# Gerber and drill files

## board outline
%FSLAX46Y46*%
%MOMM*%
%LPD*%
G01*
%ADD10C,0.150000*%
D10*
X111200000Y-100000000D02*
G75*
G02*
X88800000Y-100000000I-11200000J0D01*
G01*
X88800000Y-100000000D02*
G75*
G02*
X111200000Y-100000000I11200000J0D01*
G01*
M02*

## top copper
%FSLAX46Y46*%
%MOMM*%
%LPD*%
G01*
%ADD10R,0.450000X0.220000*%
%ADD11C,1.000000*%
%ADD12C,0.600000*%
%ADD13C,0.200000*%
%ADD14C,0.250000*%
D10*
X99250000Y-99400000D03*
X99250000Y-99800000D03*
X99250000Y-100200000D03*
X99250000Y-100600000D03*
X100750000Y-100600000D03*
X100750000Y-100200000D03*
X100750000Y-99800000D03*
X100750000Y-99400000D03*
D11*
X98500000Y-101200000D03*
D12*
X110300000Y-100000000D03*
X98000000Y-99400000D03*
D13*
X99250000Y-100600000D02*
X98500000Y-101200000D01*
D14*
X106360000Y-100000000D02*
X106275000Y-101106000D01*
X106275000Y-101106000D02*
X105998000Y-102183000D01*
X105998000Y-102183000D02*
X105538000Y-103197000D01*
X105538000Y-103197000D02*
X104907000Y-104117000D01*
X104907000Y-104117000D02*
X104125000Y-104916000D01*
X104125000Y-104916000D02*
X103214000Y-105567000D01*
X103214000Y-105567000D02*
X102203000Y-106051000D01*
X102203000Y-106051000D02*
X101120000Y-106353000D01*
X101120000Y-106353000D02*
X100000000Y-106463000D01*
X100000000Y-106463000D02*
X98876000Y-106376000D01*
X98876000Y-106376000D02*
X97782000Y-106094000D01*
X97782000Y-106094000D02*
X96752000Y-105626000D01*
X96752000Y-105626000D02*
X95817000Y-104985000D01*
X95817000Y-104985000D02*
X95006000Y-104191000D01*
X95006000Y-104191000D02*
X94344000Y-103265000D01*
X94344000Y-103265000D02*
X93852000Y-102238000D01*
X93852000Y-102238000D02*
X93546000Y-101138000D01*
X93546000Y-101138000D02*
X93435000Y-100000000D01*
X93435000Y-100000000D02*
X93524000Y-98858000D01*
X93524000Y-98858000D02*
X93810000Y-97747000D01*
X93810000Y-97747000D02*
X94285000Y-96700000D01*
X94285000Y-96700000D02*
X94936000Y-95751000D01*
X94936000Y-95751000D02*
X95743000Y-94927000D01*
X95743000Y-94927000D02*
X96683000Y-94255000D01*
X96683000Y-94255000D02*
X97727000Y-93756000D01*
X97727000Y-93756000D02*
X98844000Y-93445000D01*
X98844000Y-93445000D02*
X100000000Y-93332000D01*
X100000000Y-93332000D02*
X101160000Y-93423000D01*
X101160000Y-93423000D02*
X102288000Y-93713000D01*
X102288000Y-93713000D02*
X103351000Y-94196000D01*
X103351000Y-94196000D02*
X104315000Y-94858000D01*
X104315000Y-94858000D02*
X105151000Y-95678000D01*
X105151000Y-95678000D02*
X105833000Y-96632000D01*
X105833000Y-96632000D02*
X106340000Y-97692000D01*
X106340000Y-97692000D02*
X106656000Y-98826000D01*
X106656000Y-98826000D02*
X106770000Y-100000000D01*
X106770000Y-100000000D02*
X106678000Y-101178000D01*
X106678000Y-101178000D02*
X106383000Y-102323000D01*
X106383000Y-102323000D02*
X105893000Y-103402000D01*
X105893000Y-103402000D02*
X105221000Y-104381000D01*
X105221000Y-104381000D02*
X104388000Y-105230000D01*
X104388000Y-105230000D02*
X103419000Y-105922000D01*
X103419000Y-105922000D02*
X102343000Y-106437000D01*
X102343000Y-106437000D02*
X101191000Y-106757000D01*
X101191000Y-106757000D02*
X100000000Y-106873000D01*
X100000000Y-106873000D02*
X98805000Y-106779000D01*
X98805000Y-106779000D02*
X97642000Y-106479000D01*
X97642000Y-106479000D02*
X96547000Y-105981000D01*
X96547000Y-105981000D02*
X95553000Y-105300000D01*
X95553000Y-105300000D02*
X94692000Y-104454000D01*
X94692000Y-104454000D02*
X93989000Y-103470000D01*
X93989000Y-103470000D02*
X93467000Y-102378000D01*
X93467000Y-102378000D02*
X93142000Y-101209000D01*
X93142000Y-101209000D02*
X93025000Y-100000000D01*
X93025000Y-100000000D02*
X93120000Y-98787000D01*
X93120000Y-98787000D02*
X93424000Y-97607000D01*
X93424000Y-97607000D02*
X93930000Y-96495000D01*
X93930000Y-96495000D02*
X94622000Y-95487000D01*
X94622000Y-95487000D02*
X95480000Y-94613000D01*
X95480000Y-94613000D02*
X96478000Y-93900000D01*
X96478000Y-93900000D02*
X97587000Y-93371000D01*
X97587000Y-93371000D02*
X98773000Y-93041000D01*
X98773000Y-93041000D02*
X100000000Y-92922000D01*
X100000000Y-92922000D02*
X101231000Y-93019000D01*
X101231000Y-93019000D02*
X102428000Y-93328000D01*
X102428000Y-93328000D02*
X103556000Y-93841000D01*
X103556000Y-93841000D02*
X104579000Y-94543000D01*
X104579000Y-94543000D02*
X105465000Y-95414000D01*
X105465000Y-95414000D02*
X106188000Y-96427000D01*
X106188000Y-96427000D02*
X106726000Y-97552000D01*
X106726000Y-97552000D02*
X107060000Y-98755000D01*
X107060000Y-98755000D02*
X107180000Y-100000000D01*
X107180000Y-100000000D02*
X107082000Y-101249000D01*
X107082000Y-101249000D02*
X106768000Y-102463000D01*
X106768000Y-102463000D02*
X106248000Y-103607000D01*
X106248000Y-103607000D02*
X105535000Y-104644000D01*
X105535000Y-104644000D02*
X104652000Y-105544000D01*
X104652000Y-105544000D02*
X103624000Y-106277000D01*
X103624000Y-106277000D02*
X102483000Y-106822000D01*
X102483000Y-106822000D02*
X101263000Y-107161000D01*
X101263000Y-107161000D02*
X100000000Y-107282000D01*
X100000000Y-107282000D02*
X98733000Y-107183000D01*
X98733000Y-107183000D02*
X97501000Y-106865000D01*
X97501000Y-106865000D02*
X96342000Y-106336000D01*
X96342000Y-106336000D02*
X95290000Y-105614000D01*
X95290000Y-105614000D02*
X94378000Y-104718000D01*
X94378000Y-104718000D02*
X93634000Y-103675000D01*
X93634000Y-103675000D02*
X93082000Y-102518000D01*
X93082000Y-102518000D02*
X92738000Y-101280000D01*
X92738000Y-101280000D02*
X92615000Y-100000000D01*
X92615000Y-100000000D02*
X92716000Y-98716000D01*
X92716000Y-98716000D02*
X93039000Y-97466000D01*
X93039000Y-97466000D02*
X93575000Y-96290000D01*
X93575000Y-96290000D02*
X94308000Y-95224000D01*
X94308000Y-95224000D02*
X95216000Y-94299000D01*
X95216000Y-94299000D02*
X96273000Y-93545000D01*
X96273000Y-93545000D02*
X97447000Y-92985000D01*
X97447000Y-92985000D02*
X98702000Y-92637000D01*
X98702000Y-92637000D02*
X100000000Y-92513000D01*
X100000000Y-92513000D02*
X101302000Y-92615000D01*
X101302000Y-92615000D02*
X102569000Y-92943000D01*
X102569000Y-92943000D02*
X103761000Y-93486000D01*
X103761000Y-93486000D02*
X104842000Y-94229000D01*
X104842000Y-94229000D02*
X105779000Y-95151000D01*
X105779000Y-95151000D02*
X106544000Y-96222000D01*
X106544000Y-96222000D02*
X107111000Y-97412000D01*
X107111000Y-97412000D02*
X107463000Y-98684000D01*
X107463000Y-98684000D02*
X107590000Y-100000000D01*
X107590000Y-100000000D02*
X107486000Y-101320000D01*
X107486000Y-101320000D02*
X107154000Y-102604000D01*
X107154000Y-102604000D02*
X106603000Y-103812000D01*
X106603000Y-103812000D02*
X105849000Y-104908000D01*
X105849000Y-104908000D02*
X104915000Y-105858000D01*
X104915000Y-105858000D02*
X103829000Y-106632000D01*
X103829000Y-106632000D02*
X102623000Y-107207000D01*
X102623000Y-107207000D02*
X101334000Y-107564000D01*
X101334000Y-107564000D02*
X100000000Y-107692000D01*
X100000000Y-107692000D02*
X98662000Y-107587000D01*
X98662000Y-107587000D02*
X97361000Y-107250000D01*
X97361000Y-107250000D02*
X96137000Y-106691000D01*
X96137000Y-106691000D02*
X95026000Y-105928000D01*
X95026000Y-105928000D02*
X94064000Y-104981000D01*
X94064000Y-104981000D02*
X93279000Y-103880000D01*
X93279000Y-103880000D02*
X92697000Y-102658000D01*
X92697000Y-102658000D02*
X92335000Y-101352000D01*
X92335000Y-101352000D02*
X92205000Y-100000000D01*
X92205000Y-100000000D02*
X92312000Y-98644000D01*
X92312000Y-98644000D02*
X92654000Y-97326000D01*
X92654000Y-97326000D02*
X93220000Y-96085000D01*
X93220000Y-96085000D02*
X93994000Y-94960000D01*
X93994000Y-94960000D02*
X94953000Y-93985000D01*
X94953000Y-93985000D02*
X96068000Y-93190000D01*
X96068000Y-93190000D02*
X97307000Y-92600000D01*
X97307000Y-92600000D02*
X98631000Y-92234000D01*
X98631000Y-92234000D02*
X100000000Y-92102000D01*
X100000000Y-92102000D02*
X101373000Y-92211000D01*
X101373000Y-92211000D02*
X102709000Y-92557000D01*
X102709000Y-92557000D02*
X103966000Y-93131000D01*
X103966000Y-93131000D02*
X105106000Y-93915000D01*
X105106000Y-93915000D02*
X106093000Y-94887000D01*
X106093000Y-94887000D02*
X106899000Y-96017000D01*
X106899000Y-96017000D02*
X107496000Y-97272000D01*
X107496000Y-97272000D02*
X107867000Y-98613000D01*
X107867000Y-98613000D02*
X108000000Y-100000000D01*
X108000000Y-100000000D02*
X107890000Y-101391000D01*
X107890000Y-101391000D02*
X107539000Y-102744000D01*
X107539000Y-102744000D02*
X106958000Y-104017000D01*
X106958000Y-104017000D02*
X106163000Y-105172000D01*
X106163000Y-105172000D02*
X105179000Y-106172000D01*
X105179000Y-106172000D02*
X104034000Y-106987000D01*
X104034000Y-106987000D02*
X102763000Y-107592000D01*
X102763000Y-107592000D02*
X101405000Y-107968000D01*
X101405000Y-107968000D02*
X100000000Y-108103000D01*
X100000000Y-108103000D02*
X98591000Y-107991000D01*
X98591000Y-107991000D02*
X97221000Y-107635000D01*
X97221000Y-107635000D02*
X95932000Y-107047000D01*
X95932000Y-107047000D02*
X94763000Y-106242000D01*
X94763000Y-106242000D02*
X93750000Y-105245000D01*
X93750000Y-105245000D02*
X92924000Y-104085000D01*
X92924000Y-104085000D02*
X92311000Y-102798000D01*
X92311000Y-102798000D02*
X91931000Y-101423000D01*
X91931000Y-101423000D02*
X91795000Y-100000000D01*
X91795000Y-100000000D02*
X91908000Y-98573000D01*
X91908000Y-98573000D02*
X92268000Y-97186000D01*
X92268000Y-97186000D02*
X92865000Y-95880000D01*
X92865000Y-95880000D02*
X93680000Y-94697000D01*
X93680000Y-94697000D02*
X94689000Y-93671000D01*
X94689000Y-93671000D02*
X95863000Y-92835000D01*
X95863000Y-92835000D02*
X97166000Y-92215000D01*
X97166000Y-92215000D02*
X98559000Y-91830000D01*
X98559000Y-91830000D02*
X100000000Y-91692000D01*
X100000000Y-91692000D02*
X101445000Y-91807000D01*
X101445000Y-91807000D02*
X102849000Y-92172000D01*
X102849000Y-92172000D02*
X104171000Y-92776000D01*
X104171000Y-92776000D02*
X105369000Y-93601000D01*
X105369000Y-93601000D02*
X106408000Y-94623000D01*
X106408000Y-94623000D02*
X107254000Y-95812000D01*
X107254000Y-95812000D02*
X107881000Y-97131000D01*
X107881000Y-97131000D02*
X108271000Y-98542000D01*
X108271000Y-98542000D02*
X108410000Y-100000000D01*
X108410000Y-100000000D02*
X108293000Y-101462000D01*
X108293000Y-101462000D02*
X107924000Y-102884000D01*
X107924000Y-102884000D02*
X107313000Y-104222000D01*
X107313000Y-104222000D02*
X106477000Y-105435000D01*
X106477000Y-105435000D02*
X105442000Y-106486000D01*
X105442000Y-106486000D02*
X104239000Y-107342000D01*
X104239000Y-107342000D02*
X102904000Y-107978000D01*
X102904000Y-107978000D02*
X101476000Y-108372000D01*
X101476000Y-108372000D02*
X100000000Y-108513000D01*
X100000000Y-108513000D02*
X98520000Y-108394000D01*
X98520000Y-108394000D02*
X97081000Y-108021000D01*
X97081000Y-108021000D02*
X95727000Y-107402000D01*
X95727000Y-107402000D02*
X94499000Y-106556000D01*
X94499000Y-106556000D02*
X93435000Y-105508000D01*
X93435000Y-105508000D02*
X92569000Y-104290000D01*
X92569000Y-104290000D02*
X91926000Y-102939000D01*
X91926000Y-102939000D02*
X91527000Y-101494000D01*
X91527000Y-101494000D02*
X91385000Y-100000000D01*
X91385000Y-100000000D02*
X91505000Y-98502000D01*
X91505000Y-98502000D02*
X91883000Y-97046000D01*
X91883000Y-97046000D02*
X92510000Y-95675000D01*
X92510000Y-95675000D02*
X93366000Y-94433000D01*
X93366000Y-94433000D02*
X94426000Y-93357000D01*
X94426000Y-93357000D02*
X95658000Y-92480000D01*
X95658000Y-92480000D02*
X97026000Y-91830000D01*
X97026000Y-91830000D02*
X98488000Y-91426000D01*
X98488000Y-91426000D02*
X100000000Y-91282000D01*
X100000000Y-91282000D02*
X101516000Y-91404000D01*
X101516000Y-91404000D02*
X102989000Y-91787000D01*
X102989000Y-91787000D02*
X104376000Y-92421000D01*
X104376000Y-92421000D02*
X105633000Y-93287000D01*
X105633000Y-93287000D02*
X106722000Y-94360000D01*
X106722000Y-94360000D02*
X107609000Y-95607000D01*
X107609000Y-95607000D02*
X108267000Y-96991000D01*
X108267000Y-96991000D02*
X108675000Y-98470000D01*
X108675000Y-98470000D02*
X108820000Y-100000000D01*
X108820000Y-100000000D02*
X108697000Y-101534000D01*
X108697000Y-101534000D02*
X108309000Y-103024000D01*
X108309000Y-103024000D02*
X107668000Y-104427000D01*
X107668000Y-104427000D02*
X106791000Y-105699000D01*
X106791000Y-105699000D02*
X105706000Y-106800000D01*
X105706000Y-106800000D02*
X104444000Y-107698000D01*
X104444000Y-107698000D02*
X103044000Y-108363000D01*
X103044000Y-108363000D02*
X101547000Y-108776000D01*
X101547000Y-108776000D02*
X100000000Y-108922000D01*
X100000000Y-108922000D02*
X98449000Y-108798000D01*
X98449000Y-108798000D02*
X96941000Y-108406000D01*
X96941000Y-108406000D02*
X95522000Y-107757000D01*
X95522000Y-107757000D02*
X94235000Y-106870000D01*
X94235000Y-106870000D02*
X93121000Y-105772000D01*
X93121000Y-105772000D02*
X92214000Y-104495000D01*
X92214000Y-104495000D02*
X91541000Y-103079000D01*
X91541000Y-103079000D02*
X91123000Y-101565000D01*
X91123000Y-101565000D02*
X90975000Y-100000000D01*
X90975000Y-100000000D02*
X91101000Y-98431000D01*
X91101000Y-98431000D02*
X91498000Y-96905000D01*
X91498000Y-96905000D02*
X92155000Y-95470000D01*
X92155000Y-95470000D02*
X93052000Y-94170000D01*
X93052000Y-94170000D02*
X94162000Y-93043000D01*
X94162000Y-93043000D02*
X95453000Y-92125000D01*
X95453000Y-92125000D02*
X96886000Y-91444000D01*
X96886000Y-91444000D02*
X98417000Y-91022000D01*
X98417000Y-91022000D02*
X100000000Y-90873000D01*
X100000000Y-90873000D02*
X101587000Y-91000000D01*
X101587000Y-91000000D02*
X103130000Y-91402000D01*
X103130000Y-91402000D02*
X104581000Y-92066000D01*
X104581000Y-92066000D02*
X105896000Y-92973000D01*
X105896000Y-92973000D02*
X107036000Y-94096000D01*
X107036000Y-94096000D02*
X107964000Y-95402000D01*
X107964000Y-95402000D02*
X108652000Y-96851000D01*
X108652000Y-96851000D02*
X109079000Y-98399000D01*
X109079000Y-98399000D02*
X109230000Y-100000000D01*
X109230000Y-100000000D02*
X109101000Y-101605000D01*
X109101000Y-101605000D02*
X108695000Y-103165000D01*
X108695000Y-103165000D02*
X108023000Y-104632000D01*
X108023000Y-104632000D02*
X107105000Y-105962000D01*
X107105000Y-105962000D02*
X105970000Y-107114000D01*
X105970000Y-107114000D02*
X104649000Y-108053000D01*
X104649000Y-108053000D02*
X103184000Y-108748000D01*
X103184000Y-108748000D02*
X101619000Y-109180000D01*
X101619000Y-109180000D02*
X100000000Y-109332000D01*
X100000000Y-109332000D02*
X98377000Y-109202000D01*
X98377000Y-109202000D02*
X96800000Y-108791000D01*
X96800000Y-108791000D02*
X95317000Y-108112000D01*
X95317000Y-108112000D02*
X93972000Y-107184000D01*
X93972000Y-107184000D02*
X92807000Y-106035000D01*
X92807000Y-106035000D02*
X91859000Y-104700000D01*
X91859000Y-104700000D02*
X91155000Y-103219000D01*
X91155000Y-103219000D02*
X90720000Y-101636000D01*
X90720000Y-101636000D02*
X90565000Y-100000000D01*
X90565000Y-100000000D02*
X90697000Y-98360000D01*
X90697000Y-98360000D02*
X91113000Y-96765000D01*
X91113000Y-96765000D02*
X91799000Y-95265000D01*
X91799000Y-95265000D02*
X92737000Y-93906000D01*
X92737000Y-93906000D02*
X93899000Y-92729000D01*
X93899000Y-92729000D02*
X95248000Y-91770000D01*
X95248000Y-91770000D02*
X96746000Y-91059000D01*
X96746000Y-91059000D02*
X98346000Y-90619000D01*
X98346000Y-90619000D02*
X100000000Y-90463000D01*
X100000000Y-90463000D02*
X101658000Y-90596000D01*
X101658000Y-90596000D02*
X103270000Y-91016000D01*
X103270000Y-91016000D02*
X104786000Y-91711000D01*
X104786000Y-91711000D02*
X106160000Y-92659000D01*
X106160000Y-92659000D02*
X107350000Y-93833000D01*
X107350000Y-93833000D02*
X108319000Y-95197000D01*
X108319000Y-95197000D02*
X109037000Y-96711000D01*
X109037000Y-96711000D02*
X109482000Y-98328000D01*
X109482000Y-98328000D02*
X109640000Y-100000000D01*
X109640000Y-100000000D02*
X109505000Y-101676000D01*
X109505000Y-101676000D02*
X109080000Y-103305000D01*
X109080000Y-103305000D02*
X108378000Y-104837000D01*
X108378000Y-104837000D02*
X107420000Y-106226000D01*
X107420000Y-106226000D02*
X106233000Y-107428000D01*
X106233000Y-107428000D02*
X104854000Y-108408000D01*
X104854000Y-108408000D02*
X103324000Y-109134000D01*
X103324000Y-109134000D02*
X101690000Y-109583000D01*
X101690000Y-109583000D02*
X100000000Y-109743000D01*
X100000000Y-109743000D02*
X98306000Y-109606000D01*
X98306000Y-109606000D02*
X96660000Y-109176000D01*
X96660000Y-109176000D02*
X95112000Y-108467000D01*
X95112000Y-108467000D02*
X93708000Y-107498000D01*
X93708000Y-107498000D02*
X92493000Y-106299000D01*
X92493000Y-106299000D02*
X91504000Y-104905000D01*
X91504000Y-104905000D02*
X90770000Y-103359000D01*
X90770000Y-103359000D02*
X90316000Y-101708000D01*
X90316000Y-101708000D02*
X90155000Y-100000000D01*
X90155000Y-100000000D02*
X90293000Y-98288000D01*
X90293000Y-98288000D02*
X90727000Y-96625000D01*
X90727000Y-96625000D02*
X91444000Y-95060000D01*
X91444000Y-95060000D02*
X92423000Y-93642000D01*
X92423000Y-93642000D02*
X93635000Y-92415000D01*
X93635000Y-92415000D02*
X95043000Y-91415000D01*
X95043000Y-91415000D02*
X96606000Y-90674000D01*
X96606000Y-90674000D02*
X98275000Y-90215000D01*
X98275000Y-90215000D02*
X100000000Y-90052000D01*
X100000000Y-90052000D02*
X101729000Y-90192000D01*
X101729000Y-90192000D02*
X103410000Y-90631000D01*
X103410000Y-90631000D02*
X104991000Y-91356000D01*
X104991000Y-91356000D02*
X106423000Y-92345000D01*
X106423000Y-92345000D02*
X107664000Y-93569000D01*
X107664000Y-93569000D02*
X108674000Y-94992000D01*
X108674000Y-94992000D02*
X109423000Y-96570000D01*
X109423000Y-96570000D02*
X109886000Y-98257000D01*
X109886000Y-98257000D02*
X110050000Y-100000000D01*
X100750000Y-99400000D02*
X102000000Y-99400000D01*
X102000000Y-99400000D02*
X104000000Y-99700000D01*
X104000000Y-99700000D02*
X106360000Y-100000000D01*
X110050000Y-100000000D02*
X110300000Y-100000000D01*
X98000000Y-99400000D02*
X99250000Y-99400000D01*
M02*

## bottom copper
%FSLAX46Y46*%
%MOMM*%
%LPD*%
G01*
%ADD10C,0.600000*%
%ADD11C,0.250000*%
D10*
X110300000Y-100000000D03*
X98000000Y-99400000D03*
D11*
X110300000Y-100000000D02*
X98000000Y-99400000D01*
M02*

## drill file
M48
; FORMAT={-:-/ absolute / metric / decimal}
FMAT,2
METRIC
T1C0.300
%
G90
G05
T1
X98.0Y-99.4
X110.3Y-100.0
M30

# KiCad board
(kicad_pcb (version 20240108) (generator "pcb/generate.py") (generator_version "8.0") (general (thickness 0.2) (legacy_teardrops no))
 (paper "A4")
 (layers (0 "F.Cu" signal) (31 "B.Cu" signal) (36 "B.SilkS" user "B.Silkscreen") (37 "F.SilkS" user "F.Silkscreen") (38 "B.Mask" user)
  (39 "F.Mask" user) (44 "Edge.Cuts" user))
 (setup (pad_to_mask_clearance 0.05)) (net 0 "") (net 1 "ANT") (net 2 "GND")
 (gr_circle (center 100.00 100.00) (end 111.20 100.00) (stroke (width 0.15) (type solid)) (layer "Edge.Cuts"))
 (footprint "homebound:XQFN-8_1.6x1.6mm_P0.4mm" (layer "F.Cu") (at 100.00 100.00)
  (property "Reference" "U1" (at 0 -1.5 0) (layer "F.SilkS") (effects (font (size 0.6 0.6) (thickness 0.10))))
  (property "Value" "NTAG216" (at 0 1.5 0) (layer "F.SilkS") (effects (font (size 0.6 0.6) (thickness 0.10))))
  (pad "1" smd rect (at -0.75 -0.60) (size 0.45 0.22) (layers "F.Cu" "F.Paste" "F.Mask") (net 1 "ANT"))
  (pad "2" smd rect (at -0.75 -0.20) (size 0.45 0.22) (layers "F.Cu" "F.Paste" "F.Mask") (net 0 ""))
  (pad "3" smd rect (at -0.75 0.20) (size 0.45 0.22) (layers "F.Cu" "F.Paste" "F.Mask") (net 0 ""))
  (pad "4" smd rect (at -0.75 0.60) (size 0.45 0.22) (layers "F.Cu" "F.Paste" "F.Mask") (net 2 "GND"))
  (pad "5" smd rect (at 0.75 0.60) (size 0.45 0.22) (layers "F.Cu" "F.Paste" "F.Mask") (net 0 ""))
  (pad "6" smd rect (at 0.75 0.20) (size 0.45 0.22) (layers "F.Cu" "F.Paste" "F.Mask") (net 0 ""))
  (pad "7" smd rect (at 0.75 -0.20) (size 0.45 0.22) (layers "F.Cu" "F.Paste" "F.Mask") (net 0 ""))
  (pad "8" smd rect (at 0.75 -0.60) (size 0.45 0.22) (layers "F.Cu" "F.Paste" "F.Mask") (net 1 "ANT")))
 (segment (start 99.25 100.60) (end 98.50 101.20) (width 0.20) (layer "F.Cu") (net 2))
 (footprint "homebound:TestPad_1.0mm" (layer "F.Cu") (at 98.50 101.20)
  (pad "1" smd circle (at 0 0) (size 1.0 1.0) (layers "F.Cu" "F.Mask") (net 2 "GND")))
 (segment (start 106.360 100.000) (end 106.275 101.106) (width 0.25) (layer "F.Cu") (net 1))
 (segment (start 106.275 101.106) (end 105.998 102.183) (width 0.25) (layer "F.Cu") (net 1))
 (segment (start 105.998 102.183) (end 105.538 103.197) (width 0.25) (layer "F.Cu") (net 1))
 (segment (start 105.538 103.197) (end 104.907 104.117) (width 0.25) (layer "F.Cu") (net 1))
 (segment (start 104.907 104.117) (end 104.125 104.916) (width 0.25) (layer "F.Cu") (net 1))
 (segment (start 104.125 104.916) (end 103.214 105.567) (width 0.25) (layer "F.Cu") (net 1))
 (segment (start 103.214 105.567) (end 102.203 106.051) (width 0.25) (layer "F.Cu") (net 1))
 (segment (start 102.203 106.051) (end 101.120 106.353) (width 0.25) (layer "F.Cu") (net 1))
 (segment (start 101.120 106.353) (end 100.000 106.463) (width 0.25) (layer "F.Cu") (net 1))
 (segment (start 100.000 106.463) (end 98.876 106.376) (width 0.25) (layer "F.Cu") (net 1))
 (segment (start 98.876 106.376) (end 97.782 106.094) (width 0.25) (layer "F.Cu") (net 1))
 (segment (start 97.782 106.094) (end 96.752 105.626) (width 0.25) (layer "F.Cu") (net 1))
 (segment (start 96.752 105.626) (end 95.817 104.985) (width 0.25) (layer "F.Cu") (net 1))
 (segment (start 95.817 104.985) (end 95.006 104.191) (width 0.25) (layer "F.Cu") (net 1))
 (segment (start 95.006 104.191) (end 94.344 103.265) (width 0.25) (layer "F.Cu") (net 1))
 (segment (start 94.344 103.265) (end 93.852 102.238) (width 0.25) (layer "F.Cu") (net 1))
 (segment (start 93.852 102.238) (end 93.546 101.138) (width 0.25) (layer "F.Cu") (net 1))
 (segment (start 93.546 101.138) (end 93.435 100.000) (width 0.25) (layer "F.Cu") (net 1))
 (segment (start 93.435 100.000) (end 93.524 98.858) (width 0.25) (layer "F.Cu") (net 1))
 (segment (start 93.524 98.858) (end 93.810 97.747) (width 0.25) (layer "F.Cu") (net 1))
 (segment (start 93.810 97.747) (end 94.285 96.700) (width 0.25) (layer "F.Cu") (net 1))
 (segment (start 94.285 96.700) (end 94.936 95.751) (width 0.25) (layer "F.Cu") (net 1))
 (segment (start 94.936 95.751) (end 95.743 94.927) (width 0.25) (layer "F.Cu") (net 1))
 (segment (start 95.743 94.927) (end 96.683 94.255) (width 0.25) (layer "F.Cu") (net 1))
 (segment (start 96.683 94.255) (end 97.727 93.756) (width 0.25) (layer "F.Cu") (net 1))
 (segment (start 97.727 93.756) (end 98.844 93.445) (width 0.25) (layer "F.Cu") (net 1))
 (segment (start 98.844 93.445) (end 100.000 93.332) (width 0.25) (layer "F.Cu") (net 1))
 (segment (start 100.000 93.332) (end 101.160 93.423) (width 0.25) (layer "F.Cu") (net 1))
 (segment (start 101.160 93.423) (end 102.288 93.713) (width 0.25) (layer "F.Cu") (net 1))
 (segment (start 102.288 93.713) (end 103.351 94.196) (width 0.25) (layer "F.Cu") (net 1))
 (segment (start 103.351 94.196) (end 104.315 94.858) (width 0.25) (layer "F.Cu") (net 1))
 (segment (start 104.315 94.858) (end 105.151 95.678) (width 0.25) (layer "F.Cu") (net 1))
 (segment (start 105.151 95.678) (end 105.833 96.632) (width 0.25) (layer "F.Cu") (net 1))
 (segment (start 105.833 96.632) (end 106.340 97.692) (width 0.25) (layer "F.Cu") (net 1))
 (segment (start 106.340 97.692) (end 106.656 98.826) (width 0.25) (layer "F.Cu") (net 1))
 (segment (start 106.656 98.826) (end 106.770 100.000) (width 0.25) (layer "F.Cu") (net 1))
 (segment (start 106.770 100.000) (end 106.678 101.178) (width 0.25) (layer "F.Cu") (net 1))
 (segment (start 106.678 101.178) (end 106.383 102.323) (width 0.25) (layer "F.Cu") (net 1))
 (segment (start 106.383 102.323) (end 105.893 103.402) (width 0.25) (layer "F.Cu") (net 1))
 (segment (start 105.893 103.402) (end 105.221 104.381) (width 0.25) (layer "F.Cu") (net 1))
 (segment (start 105.221 104.381) (end 104.388 105.230) (width 0.25) (layer "F.Cu") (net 1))
 (segment (start 104.388 105.230) (end 103.419 105.922) (width 0.25) (layer "F.Cu") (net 1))
 (segment (start 103.419 105.922) (end 102.343 106.437) (width 0.25) (layer "F.Cu") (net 1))
 (segment (start 102.343 106.437) (end 101.191 106.757) (width 0.25) (layer "F.Cu") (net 1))
 (segment (start 101.191 106.757) (end 100.000 106.873) (width 0.25) (layer "F.Cu") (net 1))
 (segment (start 100.000 106.873) (end 98.805 106.779) (width 0.25) (layer "F.Cu") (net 1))
 (segment (start 98.805 106.779) (end 97.642 106.479) (width 0.25) (layer "F.Cu") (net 1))
 (segment (start 97.642 106.479) (end 96.547 105.981) (width 0.25) (layer "F.Cu") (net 1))
 (segment (start 96.547 105.981) (end 95.553 105.300) (width 0.25) (layer "F.Cu") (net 1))
 (segment (start 95.553 105.300) (end 94.692 104.454) (width 0.25) (layer "F.Cu") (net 1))
 (segment (start 94.692 104.454) (end 93.989 103.470) (width 0.25) (layer "F.Cu") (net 1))
 (segment (start 93.989 103.470) (end 93.467 102.378) (width 0.25) (layer "F.Cu") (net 1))
 (segment (start 93.467 102.378) (end 93.142 101.209) (width 0.25) (layer "F.Cu") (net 1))
 (segment (start 93.142 101.209) (end 93.025 100.000) (width 0.25) (layer "F.Cu") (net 1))
 (segment (start 93.025 100.000) (end 93.120 98.787) (width 0.25) (layer "F.Cu") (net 1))
 (segment (start 93.120 98.787) (end 93.424 97.607) (width 0.25) (layer "F.Cu") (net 1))
 (segment (start 93.424 97.607) (end 93.930 96.495) (width 0.25) (layer "F.Cu") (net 1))
 (segment (start 93.930 96.495) (end 94.622 95.487) (width 0.25) (layer "F.Cu") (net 1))
 (segment (start 94.622 95.487) (end 95.480 94.613) (width 0.25) (layer "F.Cu") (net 1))
 (segment (start 95.480 94.613) (end 96.478 93.900) (width 0.25) (layer "F.Cu") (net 1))
 (segment (start 96.478 93.900) (end 97.587 93.371) (width 0.25) (layer "F.Cu") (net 1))
 (segment (start 97.587 93.371) (end 98.773 93.041) (width 0.25) (layer "F.Cu") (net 1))
 (segment (start 98.773 93.041) (end 100.000 92.922) (width 0.25) (layer "F.Cu") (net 1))
 (segment (start 100.000 92.922) (end 101.231 93.019) (width 0.25) (layer "F.Cu") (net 1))
 (segment (start 101.231 93.019) (end 102.428 93.328) (width 0.25) (layer "F.Cu") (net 1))
 (segment (start 102.428 93.328) (end 103.556 93.841) (width 0.25) (layer "F.Cu") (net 1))
 (segment (start 103.556 93.841) (end 104.579 94.543) (width 0.25) (layer "F.Cu") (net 1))
 (segment (start 104.579 94.543) (end 105.465 95.414) (width 0.25) (layer "F.Cu") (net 1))
 (segment (start 105.465 95.414) (end 106.188 96.427) (width 0.25) (layer "F.Cu") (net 1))
 (segment (start 106.188 96.427) (end 106.726 97.552) (width 0.25) (layer "F.Cu") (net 1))
 (segment (start 106.726 97.552) (end 107.060 98.755) (width 0.25) (layer "F.Cu") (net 1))
 (segment (start 107.060 98.755) (end 107.180 100.000) (width 0.25) (layer "F.Cu") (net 1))
 (segment (start 107.180 100.000) (end 107.082 101.249) (width 0.25) (layer "F.Cu") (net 1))
 (segment (start 107.082 101.249) (end 106.768 102.463) (width 0.25) (layer "F.Cu") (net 1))
 (segment (start 106.768 102.463) (end 106.248 103.607) (width 0.25) (layer "F.Cu") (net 1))
 (segment (start 106.248 103.607) (end 105.535 104.644) (width 0.25) (layer "F.Cu") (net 1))
 (segment (start 105.535 104.644) (end 104.652 105.544) (width 0.25) (layer "F.Cu") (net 1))
 (segment (start 104.652 105.544) (end 103.624 106.277) (width 0.25) (layer "F.Cu") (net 1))
 (segment (start 103.624 106.277) (end 102.483 106.822) (width 0.25) (layer "F.Cu") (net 1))
 (segment (start 102.483 106.822) (end 101.263 107.161) (width 0.25) (layer "F.Cu") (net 1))
 (segment (start 101.263 107.161) (end 100.000 107.282) (width 0.25) (layer "F.Cu") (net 1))
 (segment (start 100.000 107.282) (end 98.733 107.183) (width 0.25) (layer "F.Cu") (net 1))
 (segment (start 98.733 107.183) (end 97.501 106.865) (width 0.25) (layer "F.Cu") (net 1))
 (segment (start 97.501 106.865) (end 96.342 106.336) (width 0.25) (layer "F.Cu") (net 1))
 (segment (start 96.342 106.336) (end 95.290 105.614) (width 0.25) (layer "F.Cu") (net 1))
 (segment (start 95.290 105.614) (end 94.378 104.718) (width 0.25) (layer "F.Cu") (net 1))
 (segment (start 94.378 104.718) (end 93.634 103.675) (width 0.25) (layer "F.Cu") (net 1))
 (segment (start 93.634 103.675) (end 93.082 102.518) (width 0.25) (layer "F.Cu") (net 1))
 (segment (start 93.082 102.518) (end 92.738 101.280) (width 0.25) (layer "F.Cu") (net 1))
 (segment (start 92.738 101.280) (end 92.615 100.000) (width 0.25) (layer "F.Cu") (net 1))
 (segment (start 92.615 100.000) (end 92.716 98.716) (width 0.25) (layer "F.Cu") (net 1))
 (segment (start 92.716 98.716) (end 93.039 97.466) (width 0.25) (layer "F.Cu") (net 1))
 (segment (start 93.039 97.466) (end 93.575 96.290) (width 0.25) (layer "F.Cu") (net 1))
 (segment (start 93.575 96.290) (end 94.308 95.224) (width 0.25) (layer "F.Cu") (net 1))
 (segment (start 94.308 95.224) (end 95.216 94.299) (width 0.25) (layer "F.Cu") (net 1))
 (segment (start 95.216 94.299) (end 96.273 93.545) (width 0.25) (layer "F.Cu") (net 1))
 (segment (start 96.273 93.545) (end 97.447 92.985) (width 0.25) (layer "F.Cu") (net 1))
 (segment (start 97.447 92.985) (end 98.702 92.637) (width 0.25) (layer "F.Cu") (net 1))
 (segment (start 98.702 92.637) (end 100.000 92.513) (width 0.25) (layer "F.Cu") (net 1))
 (segment (start 100.000 92.513) (end 101.302 92.615) (width 0.25) (layer "F.Cu") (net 1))
 (segment (start 101.302 92.615) (end 102.569 92.943) (width 0.25) (layer "F.Cu") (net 1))
 (segment (start 102.569 92.943) (end 103.761 93.486) (width 0.25) (layer "F.Cu") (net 1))
 (segment (start 103.761 93.486) (end 104.842 94.229) (width 0.25) (layer "F.Cu") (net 1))
 (segment (start 104.842 94.229) (end 105.779 95.151) (width 0.25) (layer "F.Cu") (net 1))
 (segment (start 105.779 95.151) (end 106.544 96.222) (width 0.25) (layer "F.Cu") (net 1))
 (segment (start 106.544 96.222) (end 107.111 97.412) (width 0.25) (layer "F.Cu") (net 1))
 (segment (start 107.111 97.412) (end 107.463 98.684) (width 0.25) (layer "F.Cu") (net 1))
 (segment (start 107.463 98.684) (end 107.590 100.000) (width 0.25) (layer "F.Cu") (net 1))
 (segment (start 107.590 100.000) (end 107.486 101.320) (width 0.25) (layer "F.Cu") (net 1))
 (segment (start 107.486 101.320) (end 107.154 102.604) (width 0.25) (layer "F.Cu") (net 1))
 (segment (start 107.154 102.604) (end 106.603 103.812) (width 0.25) (layer "F.Cu") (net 1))
 (segment (start 106.603 103.812) (end 105.849 104.908) (width 0.25) (layer "F.Cu") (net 1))
 (segment (start 105.849 104.908) (end 104.915 105.858) (width 0.25) (layer "F.Cu") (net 1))
 (segment (start 104.915 105.858) (end 103.829 106.632) (width 0.25) (layer "F.Cu") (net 1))
 (segment (start 103.829 106.632) (end 102.623 107.207) (width 0.25) (layer "F.Cu") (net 1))
 (segment (start 102.623 107.207) (end 101.334 107.564) (width 0.25) (layer "F.Cu") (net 1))
 (segment (start 101.334 107.564) (end 100.000 107.692) (width 0.25) (layer "F.Cu") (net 1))
 (segment (start 100.000 107.692) (end 98.662 107.587) (width 0.25) (layer "F.Cu") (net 1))
 (segment (start 98.662 107.587) (end 97.361 107.250) (width 0.25) (layer "F.Cu") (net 1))
 (segment (start 97.361 107.250) (end 96.137 106.691) (width 0.25) (layer "F.Cu") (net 1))
 (segment (start 96.137 106.691) (end 95.026 105.928) (width 0.25) (layer "F.Cu") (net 1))
 (segment (start 95.026 105.928) (end 94.064 104.981) (width 0.25) (layer "F.Cu") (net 1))
 (segment (start 94.064 104.981) (end 93.279 103.880) (width 0.25) (layer "F.Cu") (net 1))
 (segment (start 93.279 103.880) (end 92.697 102.658) (width 0.25) (layer "F.Cu") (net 1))
 (segment (start 92.697 102.658) (end 92.335 101.352) (width 0.25) (layer "F.Cu") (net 1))
 (segment (start 92.335 101.352) (end 92.205 100.000) (width 0.25) (layer "F.Cu") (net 1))
 (segment (start 92.205 100.000) (end 92.312 98.644) (width 0.25) (layer "F.Cu") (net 1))
 (segment (start 92.312 98.644) (end 92.654 97.326) (width 0.25) (layer "F.Cu") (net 1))
 (segment (start 92.654 97.326) (end 93.220 96.085) (width 0.25) (layer "F.Cu") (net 1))
 (segment (start 93.220 96.085) (end 93.994 94.960) (width 0.25) (layer "F.Cu") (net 1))
 (segment (start 93.994 94.960) (end 94.953 93.985) (width 0.25) (layer "F.Cu") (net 1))
 (segment (start 94.953 93.985) (end 96.068 93.190) (width 0.25) (layer "F.Cu") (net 1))
 (segment (start 96.068 93.190) (end 97.307 92.600) (width 0.25) (layer "F.Cu") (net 1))
 (segment (start 97.307 92.600) (end 98.631 92.234) (width 0.25) (layer "F.Cu") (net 1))
 (segment (start 98.631 92.234) (end 100.000 92.102) (width 0.25) (layer "F.Cu") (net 1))
 (segment (start 100.000 92.102) (end 101.373 92.211) (width 0.25) (layer "F.Cu") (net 1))
 (segment (start 101.373 92.211) (end 102.709 92.557) (width 0.25) (layer "F.Cu") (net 1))
 (segment (start 102.709 92.557) (end 103.966 93.131) (width 0.25) (layer "F.Cu") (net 1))
 (segment (start 103.966 93.131) (end 105.106 93.915) (width 0.25) (layer "F.Cu") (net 1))
 (segment (start 105.106 93.915) (end 106.093 94.887) (width 0.25) (layer "F.Cu") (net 1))
 (segment (start 106.093 94.887) (end 106.899 96.017) (width 0.25) (layer "F.Cu") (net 1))
 (segment (start 106.899 96.017) (end 107.496 97.272) (width 0.25) (layer "F.Cu") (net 1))
 (segment (start 107.496 97.272) (end 107.867 98.613) (width 0.25) (layer "F.Cu") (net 1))
 (segment (start 107.867 98.613) (end 108.000 100.000) (width 0.25) (layer "F.Cu") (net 1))
 (segment (start 108.000 100.000) (end 107.890 101.391) (width 0.25) (layer "F.Cu") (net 1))
 (segment (start 107.890 101.391) (end 107.539 102.744) (width 0.25) (layer "F.Cu") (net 1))
 (segment (start 107.539 102.744) (end 106.958 104.017) (width 0.25) (layer "F.Cu") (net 1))
 (segment (start 106.958 104.017) (end 106.163 105.172) (width 0.25) (layer "F.Cu") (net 1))
 (segment (start 106.163 105.172) (end 105.179 106.172) (width 0.25) (layer "F.Cu") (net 1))
 (segment (start 105.179 106.172) (end 104.034 106.987) (width 0.25) (layer "F.Cu") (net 1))
 (segment (start 104.034 106.987) (end 102.763 107.592) (width 0.25) (layer "F.Cu") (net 1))
 (segment (start 102.763 107.592) (end 101.405 107.968) (width 0.25) (layer "F.Cu") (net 1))
 (segment (start 101.405 107.968) (end 100.000 108.103) (width 0.25) (layer "F.Cu") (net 1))
 (segment (start 100.000 108.103) (end 98.591 107.991) (width 0.25) (layer "F.Cu") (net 1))
 (segment (start 98.591 107.991) (end 97.221 107.635) (width 0.25) (layer "F.Cu") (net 1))
 (segment (start 97.221 107.635) (end 95.932 107.047) (width 0.25) (layer "F.Cu") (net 1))
 (segment (start 95.932 107.047) (end 94.763 106.242) (width 0.25) (layer "F.Cu") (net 1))
 (segment (start 94.763 106.242) (end 93.750 105.245) (width 0.25) (layer "F.Cu") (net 1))
 (segment (start 93.750 105.245) (end 92.924 104.085) (width 0.25) (layer "F.Cu") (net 1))
 (segment (start 92.924 104.085) (end 92.311 102.798) (width 0.25) (layer "F.Cu") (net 1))
 (segment (start 92.311 102.798) (end 91.931 101.423) (width 0.25) (layer "F.Cu") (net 1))
 (segment (start 91.931 101.423) (end 91.795 100.000) (width 0.25) (layer "F.Cu") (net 1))
 (segment (start 91.795 100.000) (end 91.908 98.573) (width 0.25) (layer "F.Cu") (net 1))
 (segment (start 91.908 98.573) (end 92.268 97.186) (width 0.25) (layer "F.Cu") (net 1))
 (segment (start 92.268 97.186) (end 92.865 95.880) (width 0.25) (layer "F.Cu") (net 1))
 (segment (start 92.865 95.880) (end 93.680 94.697) (width 0.25) (layer "F.Cu") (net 1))
 (segment (start 93.680 94.697) (end 94.689 93.671) (width 0.25) (layer "F.Cu") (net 1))
 (segment (start 94.689 93.671) (end 95.863 92.835) (width 0.25) (layer "F.Cu") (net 1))
 (segment (start 95.863 92.835) (end 97.166 92.215) (width 0.25) (layer "F.Cu") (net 1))
 (segment (start 97.166 92.215) (end 98.559 91.830) (width 0.25) (layer "F.Cu") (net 1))
 (segment (start 98.559 91.830) (end 100.000 91.692) (width 0.25) (layer "F.Cu") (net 1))
 (segment (start 100.000 91.692) (end 101.445 91.807) (width 0.25) (layer "F.Cu") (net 1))
 (segment (start 101.445 91.807) (end 102.849 92.172) (width 0.25) (layer "F.Cu") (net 1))
 (segment (start 102.849 92.172) (end 104.171 92.776) (width 0.25) (layer "F.Cu") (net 1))
 (segment (start 104.171 92.776) (end 105.369 93.601) (width 0.25) (layer "F.Cu") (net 1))
 (segment (start 105.369 93.601) (end 106.408 94.623) (width 0.25) (layer "F.Cu") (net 1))
 (segment (start 106.408 94.623) (end 107.254 95.812) (width 0.25) (layer "F.Cu") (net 1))
 (segment (start 107.254 95.812) (end 107.881 97.131) (width 0.25) (layer "F.Cu") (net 1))
 (segment (start 107.881 97.131) (end 108.271 98.542) (width 0.25) (layer "F.Cu") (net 1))
 (segment (start 108.271 98.542) (end 108.410 100.000) (width 0.25) (layer "F.Cu") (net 1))
 (segment (start 108.410 100.000) (end 108.293 101.462) (width 0.25) (layer "F.Cu") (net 1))
 (segment (start 108.293 101.462) (end 107.924 102.884) (width 0.25) (layer "F.Cu") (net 1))
 (segment (start 107.924 102.884) (end 107.313 104.222) (width 0.25) (layer "F.Cu") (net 1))
 (segment (start 107.313 104.222) (end 106.477 105.435) (width 0.25) (layer "F.Cu") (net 1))
 (segment (start 106.477 105.435) (end 105.442 106.486) (width 0.25) (layer "F.Cu") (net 1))
 (segment (start 105.442 106.486) (end 104.239 107.342) (width 0.25) (layer "F.Cu") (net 1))
 (segment (start 104.239 107.342) (end 102.904 107.978) (width 0.25) (layer "F.Cu") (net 1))
 (segment (start 102.904 107.978) (end 101.476 108.372) (width 0.25) (layer "F.Cu") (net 1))
 (segment (start 101.476 108.372) (end 100.000 108.513) (width 0.25) (layer "F.Cu") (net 1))
 (segment (start 100.000 108.513) (end 98.520 108.394) (width 0.25) (layer "F.Cu") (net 1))
 (segment (start 98.520 108.394) (end 97.081 108.021) (width 0.25) (layer "F.Cu") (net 1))
 (segment (start 97.081 108.021) (end 95.727 107.402) (width 0.25) (layer "F.Cu") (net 1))
 (segment (start 95.727 107.402) (end 94.499 106.556) (width 0.25) (layer "F.Cu") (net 1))
 (segment (start 94.499 106.556) (end 93.435 105.508) (width 0.25) (layer "F.Cu") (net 1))
 (segment (start 93.435 105.508) (end 92.569 104.290) (width 0.25) (layer "F.Cu") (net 1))
 (segment (start 92.569 104.290) (end 91.926 102.939) (width 0.25) (layer "F.Cu") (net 1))
 (segment (start 91.926 102.939) (end 91.527 101.494) (width 0.25) (layer "F.Cu") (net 1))
 (segment (start 91.527 101.494) (end 91.385 100.000) (width 0.25) (layer "F.Cu") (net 1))
 (segment (start 91.385 100.000) (end 91.505 98.502) (width 0.25) (layer "F.Cu") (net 1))
 (segment (start 91.505 98.502) (end 91.883 97.046) (width 0.25) (layer "F.Cu") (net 1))
 (segment (start 91.883 97.046) (end 92.510 95.675) (width 0.25) (layer "F.Cu") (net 1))
 (segment (start 92.510 95.675) (end 93.366 94.433) (width 0.25) (layer "F.Cu") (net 1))
 (segment (start 93.366 94.433) (end 94.426 93.357) (width 0.25) (layer "F.Cu") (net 1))
 (segment (start 94.426 93.357) (end 95.658 92.480) (width 0.25) (layer "F.Cu") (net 1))
 (segment (start 95.658 92.480) (end 97.026 91.830) (width 0.25) (layer "F.Cu") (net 1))
 (segment (start 97.026 91.830) (end 98.488 91.426) (width 0.25) (layer "F.Cu") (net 1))
 (segment (start 98.488 91.426) (end 100.000 91.282) (width 0.25) (layer "F.Cu") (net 1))
 (segment (start 100.000 91.282) (end 101.516 91.404) (width 0.25) (layer "F.Cu") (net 1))
 (segment (start 101.516 91.404) (end 102.989 91.787) (width 0.25) (layer "F.Cu") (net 1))
 (segment (start 102.989 91.787) (end 104.376 92.421) (width 0.25) (layer "F.Cu") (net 1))
 (segment (start 104.376 92.421) (end 105.633 93.287) (width 0.25) (layer "F.Cu") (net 1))
 (segment (start 105.633 93.287) (end 106.722 94.360) (width 0.25) (layer "F.Cu") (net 1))
 (segment (start 106.722 94.360) (end 107.609 95.607) (width 0.25) (layer "F.Cu") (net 1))
 (segment (start 107.609 95.607) (end 108.267 96.991) (width 0.25) (layer "F.Cu") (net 1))
 (segment (start 108.267 96.991) (end 108.675 98.470) (width 0.25) (layer "F.Cu") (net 1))
 (segment (start 108.675 98.470) (end 108.820 100.000) (width 0.25) (layer "F.Cu") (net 1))
 (segment (start 108.820 100.000) (end 108.697 101.534) (width 0.25) (layer "F.Cu") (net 1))
 (segment (start 108.697 101.534) (end 108.309 103.024) (width 0.25) (layer "F.Cu") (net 1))
 (segment (start 108.309 103.024) (end 107.668 104.427) (width 0.25) (layer "F.Cu") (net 1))
 (segment (start 107.668 104.427) (end 106.791 105.699) (width 0.25) (layer "F.Cu") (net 1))
 (segment (start 106.791 105.699) (end 105.706 106.800) (width 0.25) (layer "F.Cu") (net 1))
 (segment (start 105.706 106.800) (end 104.444 107.698) (width 0.25) (layer "F.Cu") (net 1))
 (segment (start 104.444 107.698) (end 103.044 108.363) (width 0.25) (layer "F.Cu") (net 1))
 (segment (start 103.044 108.363) (end 101.547 108.776) (width 0.25) (layer "F.Cu") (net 1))
 (segment (start 101.547 108.776) (end 100.000 108.922) (width 0.25) (layer "F.Cu") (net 1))
 (segment (start 100.000 108.922) (end 98.449 108.798) (width 0.25) (layer "F.Cu") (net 1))
 (segment (start 98.449 108.798) (end 96.941 108.406) (width 0.25) (layer "F.Cu") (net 1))
 (segment (start 96.941 108.406) (end 95.522 107.757) (width 0.25) (layer "F.Cu") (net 1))
 (segment (start 95.522 107.757) (end 94.235 106.870) (width 0.25) (layer "F.Cu") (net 1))
 (segment (start 94.235 106.870) (end 93.121 105.772) (width 0.25) (layer "F.Cu") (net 1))
 (segment (start 93.121 105.772) (end 92.214 104.495) (width 0.25) (layer "F.Cu") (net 1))
 (segment (start 92.214 104.495) (end 91.541 103.079) (width 0.25) (layer "F.Cu") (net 1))
 (segment (start 91.541 103.079) (end 91.123 101.565) (width 0.25) (layer "F.Cu") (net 1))
 (segment (start 91.123 101.565) (end 90.975 100.000) (width 0.25) (layer "F.Cu") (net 1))
 (segment (start 90.975 100.000) (end 91.101 98.431) (width 0.25) (layer "F.Cu") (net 1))
 (segment (start 91.101 98.431) (end 91.498 96.905) (width 0.25) (layer "F.Cu") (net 1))
 (segment (start 91.498 96.905) (end 92.155 95.470) (width 0.25) (layer "F.Cu") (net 1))
 (segment (start 92.155 95.470) (end 93.052 94.170) (width 0.25) (layer "F.Cu") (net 1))
 (segment (start 93.052 94.170) (end 94.162 93.043) (width 0.25) (layer "F.Cu") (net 1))
 (segment (start 94.162 93.043) (end 95.453 92.125) (width 0.25) (layer "F.Cu") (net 1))
 (segment (start 95.453 92.125) (end 96.886 91.444) (width 0.25) (layer "F.Cu") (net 1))
 (segment (start 96.886 91.444) (end 98.417 91.022) (width 0.25) (layer "F.Cu") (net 1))
 (segment (start 98.417 91.022) (end 100.000 90.873) (width 0.25) (layer "F.Cu") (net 1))
 (segment (start 100.000 90.873) (end 101.587 91.000) (width 0.25) (layer "F.Cu") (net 1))
 (segment (start 101.587 91.000) (end 103.130 91.402) (width 0.25) (layer "F.Cu") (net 1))
 (segment (start 103.130 91.402) (end 104.581 92.066) (width 0.25) (layer "F.Cu") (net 1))
 (segment (start 104.581 92.066) (end 105.896 92.973) (width 0.25) (layer "F.Cu") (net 1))
 (segment (start 105.896 92.973) (end 107.036 94.096) (width 0.25) (layer "F.Cu") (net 1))
 (segment (start 107.036 94.096) (end 107.964 95.402) (width 0.25) (layer "F.Cu") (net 1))
 (segment (start 107.964 95.402) (end 108.652 96.851) (width 0.25) (layer "F.Cu") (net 1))
 (segment (start 108.652 96.851) (end 109.079 98.399) (width 0.25) (layer "F.Cu") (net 1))
 (segment (start 109.079 98.399) (end 109.230 100.000) (width 0.25) (layer "F.Cu") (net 1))
 (segment (start 109.230 100.000) (end 109.101 101.605) (width 0.25) (layer "F.Cu") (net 1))
 (segment (start 109.101 101.605) (end 108.695 103.165) (width 0.25) (layer "F.Cu") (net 1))
 (segment (start 108.695 103.165) (end 108.023 104.632) (width 0.25) (layer "F.Cu") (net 1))
 (segment (start 108.023 104.632) (end 107.105 105.962) (width 0.25) (layer "F.Cu") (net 1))
 (segment (start 107.105 105.962) (end 105.970 107.114) (width 0.25) (layer "F.Cu") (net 1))
 (segment (start 105.970 107.114) (end 104.649 108.053) (width 0.25) (layer "F.Cu") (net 1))
 (segment (start 104.649 108.053) (end 103.184 108.748) (width 0.25) (layer "F.Cu") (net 1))
 (segment (start 103.184 108.748) (end 101.619 109.180) (width 0.25) (layer "F.Cu") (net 1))
 (segment (start 101.619 109.180) (end 100.000 109.332) (width 0.25) (layer "F.Cu") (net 1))
 (segment (start 100.000 109.332) (end 98.377 109.202) (width 0.25) (layer "F.Cu") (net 1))
 (segment (start 98.377 109.202) (end 96.800 108.791) (width 0.25) (layer "F.Cu") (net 1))
 (segment (start 96.800 108.791) (end 95.317 108.112) (width 0.25) (layer "F.Cu") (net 1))
 (segment (start 95.317 108.112) (end 93.972 107.184) (width 0.25) (layer "F.Cu") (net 1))
 (segment (start 93.972 107.184) (end 92.807 106.035) (width 0.25) (layer "F.Cu") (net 1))
 (segment (start 92.807 106.035) (end 91.859 104.700) (width 0.25) (layer "F.Cu") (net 1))
 (segment (start 91.859 104.700) (end 91.155 103.219) (width 0.25) (layer "F.Cu") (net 1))
 (segment (start 91.155 103.219) (end 90.720 101.636) (width 0.25) (layer "F.Cu") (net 1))
 (segment (start 90.720 101.636) (end 90.565 100.000) (width 0.25) (layer "F.Cu") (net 1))
 (segment (start 90.565 100.000) (end 90.697 98.360) (width 0.25) (layer "F.Cu") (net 1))
 (segment (start 90.697 98.360) (end 91.113 96.765) (width 0.25) (layer "F.Cu") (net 1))
 (segment (start 91.113 96.765) (end 91.799 95.265) (width 0.25) (layer "F.Cu") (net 1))
 (segment (start 91.799 95.265) (end 92.737 93.906) (width 0.25) (layer "F.Cu") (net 1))
 (segment (start 92.737 93.906) (end 93.899 92.729) (width 0.25) (layer "F.Cu") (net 1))
 (segment (start 93.899 92.729) (end 95.248 91.770) (width 0.25) (layer "F.Cu") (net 1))
 (segment (start 95.248 91.770) (end 96.746 91.059) (width 0.25) (layer "F.Cu") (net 1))
 (segment (start 96.746 91.059) (end 98.346 90.619) (width 0.25) (layer "F.Cu") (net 1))
 (segment (start 98.346 90.619) (end 100.000 90.463) (width 0.25) (layer "F.Cu") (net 1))
 (segment (start 100.000 90.463) (end 101.658 90.596) (width 0.25) (layer "F.Cu") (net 1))
 (segment (start 101.658 90.596) (end 103.270 91.016) (width 0.25) (layer "F.Cu") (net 1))
 (segment (start 103.270 91.016) (end 104.786 91.711) (width 0.25) (layer "F.Cu") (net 1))
 (segment (start 104.786 91.711) (end 106.160 92.659) (width 0.25) (layer "F.Cu") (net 1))
 (segment (start 106.160 92.659) (end 107.350 93.833) (width 0.25) (layer "F.Cu") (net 1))
 (segment (start 107.350 93.833) (end 108.319 95.197) (width 0.25) (layer "F.Cu") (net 1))
 (segment (start 108.319 95.197) (end 109.037 96.711) (width 0.25) (layer "F.Cu") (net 1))
 (segment (start 109.037 96.711) (end 109.482 98.328) (width 0.25) (layer "F.Cu") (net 1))
 (segment (start 109.482 98.328) (end 109.640 100.000) (width 0.25) (layer "F.Cu") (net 1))
 (segment (start 109.640 100.000) (end 109.505 101.676) (width 0.25) (layer "F.Cu") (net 1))
 (segment (start 109.505 101.676) (end 109.080 103.305) (width 0.25) (layer "F.Cu") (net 1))
 (segment (start 109.080 103.305) (end 108.378 104.837) (width 0.25) (layer "F.Cu") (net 1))
 (segment (start 108.378 104.837) (end 107.420 106.226) (width 0.25) (layer "F.Cu") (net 1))
 (segment (start 107.420 106.226) (end 106.233 107.428) (width 0.25) (layer "F.Cu") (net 1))
 (segment (start 106.233 107.428) (end 104.854 108.408) (width 0.25) (layer "F.Cu") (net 1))
 (segment (start 104.854 108.408) (end 103.324 109.134) (width 0.25) (layer "F.Cu") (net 1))
 (segment (start 103.324 109.134) (end 101.690 109.583) (width 0.25) (layer "F.Cu") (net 1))
 (segment (start 101.690 109.583) (end 100.000 109.743) (width 0.25) (layer "F.Cu") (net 1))
 (segment (start 100.000 109.743) (end 98.306 109.606) (width 0.25) (layer "F.Cu") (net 1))
 (segment (start 98.306 109.606) (end 96.660 109.176) (width 0.25) (layer "F.Cu") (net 1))
 (segment (start 96.660 109.176) (end 95.112 108.467) (width 0.25) (layer "F.Cu") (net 1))
 (segment (start 95.112 108.467) (end 93.708 107.498) (width 0.25) (layer "F.Cu") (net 1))
 (segment (start 93.708 107.498) (end 92.493 106.299) (width 0.25) (layer "F.Cu") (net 1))
 (segment (start 92.493 106.299) (end 91.504 104.905) (width 0.25) (layer "F.Cu") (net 1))
 (segment (start 91.504 104.905) (end 90.770 103.359) (width 0.25) (layer "F.Cu") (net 1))
 (segment (start 90.770 103.359) (end 90.316 101.708) (width 0.25) (layer "F.Cu") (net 1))
 (segment (start 90.316 101.708) (end 90.155 100.000) (width 0.25) (layer "F.Cu") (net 1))
 (segment (start 90.155 100.000) (end 90.293 98.288) (width 0.25) (layer "F.Cu") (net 1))
 (segment (start 90.293 98.288) (end 90.727 96.625) (width 0.25) (layer "F.Cu") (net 1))
 (segment (start 90.727 96.625) (end 91.444 95.060) (width 0.25) (layer "F.Cu") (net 1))
 (segment (start 91.444 95.060) (end 92.423 93.642) (width 0.25) (layer "F.Cu") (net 1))
 (segment (start 92.423 93.642) (end 93.635 92.415) (width 0.25) (layer "F.Cu") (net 1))
 (segment (start 93.635 92.415) (end 95.043 91.415) (width 0.25) (layer "F.Cu") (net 1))
 (segment (start 95.043 91.415) (end 96.606 90.674) (width 0.25) (layer "F.Cu") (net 1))
 (segment (start 96.606 90.674) (end 98.275 90.215) (width 0.25) (layer "F.Cu") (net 1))
 (segment (start 98.275 90.215) (end 100.000 90.052) (width 0.25) (layer "F.Cu") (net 1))
 (segment (start 100.000 90.052) (end 101.729 90.192) (width 0.25) (layer "F.Cu") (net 1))
 (segment (start 101.729 90.192) (end 103.410 90.631) (width 0.25) (layer "F.Cu") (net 1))
 (segment (start 103.410 90.631) (end 104.991 91.356) (width 0.25) (layer "F.Cu") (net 1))
 (segment (start 104.991 91.356) (end 106.423 92.345) (width 0.25) (layer "F.Cu") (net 1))
 (segment (start 106.423 92.345) (end 107.664 93.569) (width 0.25) (layer "F.Cu") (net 1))
 (segment (start 107.664 93.569) (end 108.674 94.992) (width 0.25) (layer "F.Cu") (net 1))
 (segment (start 108.674 94.992) (end 109.423 96.570) (width 0.25) (layer "F.Cu") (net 1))
 (segment (start 109.423 96.570) (end 109.886 98.257) (width 0.25) (layer "F.Cu") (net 1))
 (segment (start 109.886 98.257) (end 110.050 100.000) (width 0.25) (layer "F.Cu") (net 1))
 (segment (start 100.750 99.400) (end 102.000 99.400) (width 0.25) (layer "F.Cu") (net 1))
 (segment (start 102.000 99.400) (end 104.000 99.700) (width 0.25) (layer "F.Cu") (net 1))
 (segment (start 104.000 99.700) (end 106.360 100.000) (width 0.25) (layer "F.Cu") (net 1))
 (segment (start 110.050 100.000) (end 110.300 100.000) (width 0.25) (layer "F.Cu") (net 1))
 (via (at 110.300 100.000) (size 0.60) (drill 0.30) (layers "F.Cu" "B.Cu") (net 1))
 (segment (start 110.300 100.000) (end 98.000 99.400) (width 0.25) (layer "B.Cu") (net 1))
 (via (at 98.000 99.400) (size 0.60) (drill 0.30) (layers "F.Cu" "B.Cu") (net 1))
 (segment (start 98.000 99.400) (end 99.250 99.400) (width 0.25) (layer "F.Cu") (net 1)))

